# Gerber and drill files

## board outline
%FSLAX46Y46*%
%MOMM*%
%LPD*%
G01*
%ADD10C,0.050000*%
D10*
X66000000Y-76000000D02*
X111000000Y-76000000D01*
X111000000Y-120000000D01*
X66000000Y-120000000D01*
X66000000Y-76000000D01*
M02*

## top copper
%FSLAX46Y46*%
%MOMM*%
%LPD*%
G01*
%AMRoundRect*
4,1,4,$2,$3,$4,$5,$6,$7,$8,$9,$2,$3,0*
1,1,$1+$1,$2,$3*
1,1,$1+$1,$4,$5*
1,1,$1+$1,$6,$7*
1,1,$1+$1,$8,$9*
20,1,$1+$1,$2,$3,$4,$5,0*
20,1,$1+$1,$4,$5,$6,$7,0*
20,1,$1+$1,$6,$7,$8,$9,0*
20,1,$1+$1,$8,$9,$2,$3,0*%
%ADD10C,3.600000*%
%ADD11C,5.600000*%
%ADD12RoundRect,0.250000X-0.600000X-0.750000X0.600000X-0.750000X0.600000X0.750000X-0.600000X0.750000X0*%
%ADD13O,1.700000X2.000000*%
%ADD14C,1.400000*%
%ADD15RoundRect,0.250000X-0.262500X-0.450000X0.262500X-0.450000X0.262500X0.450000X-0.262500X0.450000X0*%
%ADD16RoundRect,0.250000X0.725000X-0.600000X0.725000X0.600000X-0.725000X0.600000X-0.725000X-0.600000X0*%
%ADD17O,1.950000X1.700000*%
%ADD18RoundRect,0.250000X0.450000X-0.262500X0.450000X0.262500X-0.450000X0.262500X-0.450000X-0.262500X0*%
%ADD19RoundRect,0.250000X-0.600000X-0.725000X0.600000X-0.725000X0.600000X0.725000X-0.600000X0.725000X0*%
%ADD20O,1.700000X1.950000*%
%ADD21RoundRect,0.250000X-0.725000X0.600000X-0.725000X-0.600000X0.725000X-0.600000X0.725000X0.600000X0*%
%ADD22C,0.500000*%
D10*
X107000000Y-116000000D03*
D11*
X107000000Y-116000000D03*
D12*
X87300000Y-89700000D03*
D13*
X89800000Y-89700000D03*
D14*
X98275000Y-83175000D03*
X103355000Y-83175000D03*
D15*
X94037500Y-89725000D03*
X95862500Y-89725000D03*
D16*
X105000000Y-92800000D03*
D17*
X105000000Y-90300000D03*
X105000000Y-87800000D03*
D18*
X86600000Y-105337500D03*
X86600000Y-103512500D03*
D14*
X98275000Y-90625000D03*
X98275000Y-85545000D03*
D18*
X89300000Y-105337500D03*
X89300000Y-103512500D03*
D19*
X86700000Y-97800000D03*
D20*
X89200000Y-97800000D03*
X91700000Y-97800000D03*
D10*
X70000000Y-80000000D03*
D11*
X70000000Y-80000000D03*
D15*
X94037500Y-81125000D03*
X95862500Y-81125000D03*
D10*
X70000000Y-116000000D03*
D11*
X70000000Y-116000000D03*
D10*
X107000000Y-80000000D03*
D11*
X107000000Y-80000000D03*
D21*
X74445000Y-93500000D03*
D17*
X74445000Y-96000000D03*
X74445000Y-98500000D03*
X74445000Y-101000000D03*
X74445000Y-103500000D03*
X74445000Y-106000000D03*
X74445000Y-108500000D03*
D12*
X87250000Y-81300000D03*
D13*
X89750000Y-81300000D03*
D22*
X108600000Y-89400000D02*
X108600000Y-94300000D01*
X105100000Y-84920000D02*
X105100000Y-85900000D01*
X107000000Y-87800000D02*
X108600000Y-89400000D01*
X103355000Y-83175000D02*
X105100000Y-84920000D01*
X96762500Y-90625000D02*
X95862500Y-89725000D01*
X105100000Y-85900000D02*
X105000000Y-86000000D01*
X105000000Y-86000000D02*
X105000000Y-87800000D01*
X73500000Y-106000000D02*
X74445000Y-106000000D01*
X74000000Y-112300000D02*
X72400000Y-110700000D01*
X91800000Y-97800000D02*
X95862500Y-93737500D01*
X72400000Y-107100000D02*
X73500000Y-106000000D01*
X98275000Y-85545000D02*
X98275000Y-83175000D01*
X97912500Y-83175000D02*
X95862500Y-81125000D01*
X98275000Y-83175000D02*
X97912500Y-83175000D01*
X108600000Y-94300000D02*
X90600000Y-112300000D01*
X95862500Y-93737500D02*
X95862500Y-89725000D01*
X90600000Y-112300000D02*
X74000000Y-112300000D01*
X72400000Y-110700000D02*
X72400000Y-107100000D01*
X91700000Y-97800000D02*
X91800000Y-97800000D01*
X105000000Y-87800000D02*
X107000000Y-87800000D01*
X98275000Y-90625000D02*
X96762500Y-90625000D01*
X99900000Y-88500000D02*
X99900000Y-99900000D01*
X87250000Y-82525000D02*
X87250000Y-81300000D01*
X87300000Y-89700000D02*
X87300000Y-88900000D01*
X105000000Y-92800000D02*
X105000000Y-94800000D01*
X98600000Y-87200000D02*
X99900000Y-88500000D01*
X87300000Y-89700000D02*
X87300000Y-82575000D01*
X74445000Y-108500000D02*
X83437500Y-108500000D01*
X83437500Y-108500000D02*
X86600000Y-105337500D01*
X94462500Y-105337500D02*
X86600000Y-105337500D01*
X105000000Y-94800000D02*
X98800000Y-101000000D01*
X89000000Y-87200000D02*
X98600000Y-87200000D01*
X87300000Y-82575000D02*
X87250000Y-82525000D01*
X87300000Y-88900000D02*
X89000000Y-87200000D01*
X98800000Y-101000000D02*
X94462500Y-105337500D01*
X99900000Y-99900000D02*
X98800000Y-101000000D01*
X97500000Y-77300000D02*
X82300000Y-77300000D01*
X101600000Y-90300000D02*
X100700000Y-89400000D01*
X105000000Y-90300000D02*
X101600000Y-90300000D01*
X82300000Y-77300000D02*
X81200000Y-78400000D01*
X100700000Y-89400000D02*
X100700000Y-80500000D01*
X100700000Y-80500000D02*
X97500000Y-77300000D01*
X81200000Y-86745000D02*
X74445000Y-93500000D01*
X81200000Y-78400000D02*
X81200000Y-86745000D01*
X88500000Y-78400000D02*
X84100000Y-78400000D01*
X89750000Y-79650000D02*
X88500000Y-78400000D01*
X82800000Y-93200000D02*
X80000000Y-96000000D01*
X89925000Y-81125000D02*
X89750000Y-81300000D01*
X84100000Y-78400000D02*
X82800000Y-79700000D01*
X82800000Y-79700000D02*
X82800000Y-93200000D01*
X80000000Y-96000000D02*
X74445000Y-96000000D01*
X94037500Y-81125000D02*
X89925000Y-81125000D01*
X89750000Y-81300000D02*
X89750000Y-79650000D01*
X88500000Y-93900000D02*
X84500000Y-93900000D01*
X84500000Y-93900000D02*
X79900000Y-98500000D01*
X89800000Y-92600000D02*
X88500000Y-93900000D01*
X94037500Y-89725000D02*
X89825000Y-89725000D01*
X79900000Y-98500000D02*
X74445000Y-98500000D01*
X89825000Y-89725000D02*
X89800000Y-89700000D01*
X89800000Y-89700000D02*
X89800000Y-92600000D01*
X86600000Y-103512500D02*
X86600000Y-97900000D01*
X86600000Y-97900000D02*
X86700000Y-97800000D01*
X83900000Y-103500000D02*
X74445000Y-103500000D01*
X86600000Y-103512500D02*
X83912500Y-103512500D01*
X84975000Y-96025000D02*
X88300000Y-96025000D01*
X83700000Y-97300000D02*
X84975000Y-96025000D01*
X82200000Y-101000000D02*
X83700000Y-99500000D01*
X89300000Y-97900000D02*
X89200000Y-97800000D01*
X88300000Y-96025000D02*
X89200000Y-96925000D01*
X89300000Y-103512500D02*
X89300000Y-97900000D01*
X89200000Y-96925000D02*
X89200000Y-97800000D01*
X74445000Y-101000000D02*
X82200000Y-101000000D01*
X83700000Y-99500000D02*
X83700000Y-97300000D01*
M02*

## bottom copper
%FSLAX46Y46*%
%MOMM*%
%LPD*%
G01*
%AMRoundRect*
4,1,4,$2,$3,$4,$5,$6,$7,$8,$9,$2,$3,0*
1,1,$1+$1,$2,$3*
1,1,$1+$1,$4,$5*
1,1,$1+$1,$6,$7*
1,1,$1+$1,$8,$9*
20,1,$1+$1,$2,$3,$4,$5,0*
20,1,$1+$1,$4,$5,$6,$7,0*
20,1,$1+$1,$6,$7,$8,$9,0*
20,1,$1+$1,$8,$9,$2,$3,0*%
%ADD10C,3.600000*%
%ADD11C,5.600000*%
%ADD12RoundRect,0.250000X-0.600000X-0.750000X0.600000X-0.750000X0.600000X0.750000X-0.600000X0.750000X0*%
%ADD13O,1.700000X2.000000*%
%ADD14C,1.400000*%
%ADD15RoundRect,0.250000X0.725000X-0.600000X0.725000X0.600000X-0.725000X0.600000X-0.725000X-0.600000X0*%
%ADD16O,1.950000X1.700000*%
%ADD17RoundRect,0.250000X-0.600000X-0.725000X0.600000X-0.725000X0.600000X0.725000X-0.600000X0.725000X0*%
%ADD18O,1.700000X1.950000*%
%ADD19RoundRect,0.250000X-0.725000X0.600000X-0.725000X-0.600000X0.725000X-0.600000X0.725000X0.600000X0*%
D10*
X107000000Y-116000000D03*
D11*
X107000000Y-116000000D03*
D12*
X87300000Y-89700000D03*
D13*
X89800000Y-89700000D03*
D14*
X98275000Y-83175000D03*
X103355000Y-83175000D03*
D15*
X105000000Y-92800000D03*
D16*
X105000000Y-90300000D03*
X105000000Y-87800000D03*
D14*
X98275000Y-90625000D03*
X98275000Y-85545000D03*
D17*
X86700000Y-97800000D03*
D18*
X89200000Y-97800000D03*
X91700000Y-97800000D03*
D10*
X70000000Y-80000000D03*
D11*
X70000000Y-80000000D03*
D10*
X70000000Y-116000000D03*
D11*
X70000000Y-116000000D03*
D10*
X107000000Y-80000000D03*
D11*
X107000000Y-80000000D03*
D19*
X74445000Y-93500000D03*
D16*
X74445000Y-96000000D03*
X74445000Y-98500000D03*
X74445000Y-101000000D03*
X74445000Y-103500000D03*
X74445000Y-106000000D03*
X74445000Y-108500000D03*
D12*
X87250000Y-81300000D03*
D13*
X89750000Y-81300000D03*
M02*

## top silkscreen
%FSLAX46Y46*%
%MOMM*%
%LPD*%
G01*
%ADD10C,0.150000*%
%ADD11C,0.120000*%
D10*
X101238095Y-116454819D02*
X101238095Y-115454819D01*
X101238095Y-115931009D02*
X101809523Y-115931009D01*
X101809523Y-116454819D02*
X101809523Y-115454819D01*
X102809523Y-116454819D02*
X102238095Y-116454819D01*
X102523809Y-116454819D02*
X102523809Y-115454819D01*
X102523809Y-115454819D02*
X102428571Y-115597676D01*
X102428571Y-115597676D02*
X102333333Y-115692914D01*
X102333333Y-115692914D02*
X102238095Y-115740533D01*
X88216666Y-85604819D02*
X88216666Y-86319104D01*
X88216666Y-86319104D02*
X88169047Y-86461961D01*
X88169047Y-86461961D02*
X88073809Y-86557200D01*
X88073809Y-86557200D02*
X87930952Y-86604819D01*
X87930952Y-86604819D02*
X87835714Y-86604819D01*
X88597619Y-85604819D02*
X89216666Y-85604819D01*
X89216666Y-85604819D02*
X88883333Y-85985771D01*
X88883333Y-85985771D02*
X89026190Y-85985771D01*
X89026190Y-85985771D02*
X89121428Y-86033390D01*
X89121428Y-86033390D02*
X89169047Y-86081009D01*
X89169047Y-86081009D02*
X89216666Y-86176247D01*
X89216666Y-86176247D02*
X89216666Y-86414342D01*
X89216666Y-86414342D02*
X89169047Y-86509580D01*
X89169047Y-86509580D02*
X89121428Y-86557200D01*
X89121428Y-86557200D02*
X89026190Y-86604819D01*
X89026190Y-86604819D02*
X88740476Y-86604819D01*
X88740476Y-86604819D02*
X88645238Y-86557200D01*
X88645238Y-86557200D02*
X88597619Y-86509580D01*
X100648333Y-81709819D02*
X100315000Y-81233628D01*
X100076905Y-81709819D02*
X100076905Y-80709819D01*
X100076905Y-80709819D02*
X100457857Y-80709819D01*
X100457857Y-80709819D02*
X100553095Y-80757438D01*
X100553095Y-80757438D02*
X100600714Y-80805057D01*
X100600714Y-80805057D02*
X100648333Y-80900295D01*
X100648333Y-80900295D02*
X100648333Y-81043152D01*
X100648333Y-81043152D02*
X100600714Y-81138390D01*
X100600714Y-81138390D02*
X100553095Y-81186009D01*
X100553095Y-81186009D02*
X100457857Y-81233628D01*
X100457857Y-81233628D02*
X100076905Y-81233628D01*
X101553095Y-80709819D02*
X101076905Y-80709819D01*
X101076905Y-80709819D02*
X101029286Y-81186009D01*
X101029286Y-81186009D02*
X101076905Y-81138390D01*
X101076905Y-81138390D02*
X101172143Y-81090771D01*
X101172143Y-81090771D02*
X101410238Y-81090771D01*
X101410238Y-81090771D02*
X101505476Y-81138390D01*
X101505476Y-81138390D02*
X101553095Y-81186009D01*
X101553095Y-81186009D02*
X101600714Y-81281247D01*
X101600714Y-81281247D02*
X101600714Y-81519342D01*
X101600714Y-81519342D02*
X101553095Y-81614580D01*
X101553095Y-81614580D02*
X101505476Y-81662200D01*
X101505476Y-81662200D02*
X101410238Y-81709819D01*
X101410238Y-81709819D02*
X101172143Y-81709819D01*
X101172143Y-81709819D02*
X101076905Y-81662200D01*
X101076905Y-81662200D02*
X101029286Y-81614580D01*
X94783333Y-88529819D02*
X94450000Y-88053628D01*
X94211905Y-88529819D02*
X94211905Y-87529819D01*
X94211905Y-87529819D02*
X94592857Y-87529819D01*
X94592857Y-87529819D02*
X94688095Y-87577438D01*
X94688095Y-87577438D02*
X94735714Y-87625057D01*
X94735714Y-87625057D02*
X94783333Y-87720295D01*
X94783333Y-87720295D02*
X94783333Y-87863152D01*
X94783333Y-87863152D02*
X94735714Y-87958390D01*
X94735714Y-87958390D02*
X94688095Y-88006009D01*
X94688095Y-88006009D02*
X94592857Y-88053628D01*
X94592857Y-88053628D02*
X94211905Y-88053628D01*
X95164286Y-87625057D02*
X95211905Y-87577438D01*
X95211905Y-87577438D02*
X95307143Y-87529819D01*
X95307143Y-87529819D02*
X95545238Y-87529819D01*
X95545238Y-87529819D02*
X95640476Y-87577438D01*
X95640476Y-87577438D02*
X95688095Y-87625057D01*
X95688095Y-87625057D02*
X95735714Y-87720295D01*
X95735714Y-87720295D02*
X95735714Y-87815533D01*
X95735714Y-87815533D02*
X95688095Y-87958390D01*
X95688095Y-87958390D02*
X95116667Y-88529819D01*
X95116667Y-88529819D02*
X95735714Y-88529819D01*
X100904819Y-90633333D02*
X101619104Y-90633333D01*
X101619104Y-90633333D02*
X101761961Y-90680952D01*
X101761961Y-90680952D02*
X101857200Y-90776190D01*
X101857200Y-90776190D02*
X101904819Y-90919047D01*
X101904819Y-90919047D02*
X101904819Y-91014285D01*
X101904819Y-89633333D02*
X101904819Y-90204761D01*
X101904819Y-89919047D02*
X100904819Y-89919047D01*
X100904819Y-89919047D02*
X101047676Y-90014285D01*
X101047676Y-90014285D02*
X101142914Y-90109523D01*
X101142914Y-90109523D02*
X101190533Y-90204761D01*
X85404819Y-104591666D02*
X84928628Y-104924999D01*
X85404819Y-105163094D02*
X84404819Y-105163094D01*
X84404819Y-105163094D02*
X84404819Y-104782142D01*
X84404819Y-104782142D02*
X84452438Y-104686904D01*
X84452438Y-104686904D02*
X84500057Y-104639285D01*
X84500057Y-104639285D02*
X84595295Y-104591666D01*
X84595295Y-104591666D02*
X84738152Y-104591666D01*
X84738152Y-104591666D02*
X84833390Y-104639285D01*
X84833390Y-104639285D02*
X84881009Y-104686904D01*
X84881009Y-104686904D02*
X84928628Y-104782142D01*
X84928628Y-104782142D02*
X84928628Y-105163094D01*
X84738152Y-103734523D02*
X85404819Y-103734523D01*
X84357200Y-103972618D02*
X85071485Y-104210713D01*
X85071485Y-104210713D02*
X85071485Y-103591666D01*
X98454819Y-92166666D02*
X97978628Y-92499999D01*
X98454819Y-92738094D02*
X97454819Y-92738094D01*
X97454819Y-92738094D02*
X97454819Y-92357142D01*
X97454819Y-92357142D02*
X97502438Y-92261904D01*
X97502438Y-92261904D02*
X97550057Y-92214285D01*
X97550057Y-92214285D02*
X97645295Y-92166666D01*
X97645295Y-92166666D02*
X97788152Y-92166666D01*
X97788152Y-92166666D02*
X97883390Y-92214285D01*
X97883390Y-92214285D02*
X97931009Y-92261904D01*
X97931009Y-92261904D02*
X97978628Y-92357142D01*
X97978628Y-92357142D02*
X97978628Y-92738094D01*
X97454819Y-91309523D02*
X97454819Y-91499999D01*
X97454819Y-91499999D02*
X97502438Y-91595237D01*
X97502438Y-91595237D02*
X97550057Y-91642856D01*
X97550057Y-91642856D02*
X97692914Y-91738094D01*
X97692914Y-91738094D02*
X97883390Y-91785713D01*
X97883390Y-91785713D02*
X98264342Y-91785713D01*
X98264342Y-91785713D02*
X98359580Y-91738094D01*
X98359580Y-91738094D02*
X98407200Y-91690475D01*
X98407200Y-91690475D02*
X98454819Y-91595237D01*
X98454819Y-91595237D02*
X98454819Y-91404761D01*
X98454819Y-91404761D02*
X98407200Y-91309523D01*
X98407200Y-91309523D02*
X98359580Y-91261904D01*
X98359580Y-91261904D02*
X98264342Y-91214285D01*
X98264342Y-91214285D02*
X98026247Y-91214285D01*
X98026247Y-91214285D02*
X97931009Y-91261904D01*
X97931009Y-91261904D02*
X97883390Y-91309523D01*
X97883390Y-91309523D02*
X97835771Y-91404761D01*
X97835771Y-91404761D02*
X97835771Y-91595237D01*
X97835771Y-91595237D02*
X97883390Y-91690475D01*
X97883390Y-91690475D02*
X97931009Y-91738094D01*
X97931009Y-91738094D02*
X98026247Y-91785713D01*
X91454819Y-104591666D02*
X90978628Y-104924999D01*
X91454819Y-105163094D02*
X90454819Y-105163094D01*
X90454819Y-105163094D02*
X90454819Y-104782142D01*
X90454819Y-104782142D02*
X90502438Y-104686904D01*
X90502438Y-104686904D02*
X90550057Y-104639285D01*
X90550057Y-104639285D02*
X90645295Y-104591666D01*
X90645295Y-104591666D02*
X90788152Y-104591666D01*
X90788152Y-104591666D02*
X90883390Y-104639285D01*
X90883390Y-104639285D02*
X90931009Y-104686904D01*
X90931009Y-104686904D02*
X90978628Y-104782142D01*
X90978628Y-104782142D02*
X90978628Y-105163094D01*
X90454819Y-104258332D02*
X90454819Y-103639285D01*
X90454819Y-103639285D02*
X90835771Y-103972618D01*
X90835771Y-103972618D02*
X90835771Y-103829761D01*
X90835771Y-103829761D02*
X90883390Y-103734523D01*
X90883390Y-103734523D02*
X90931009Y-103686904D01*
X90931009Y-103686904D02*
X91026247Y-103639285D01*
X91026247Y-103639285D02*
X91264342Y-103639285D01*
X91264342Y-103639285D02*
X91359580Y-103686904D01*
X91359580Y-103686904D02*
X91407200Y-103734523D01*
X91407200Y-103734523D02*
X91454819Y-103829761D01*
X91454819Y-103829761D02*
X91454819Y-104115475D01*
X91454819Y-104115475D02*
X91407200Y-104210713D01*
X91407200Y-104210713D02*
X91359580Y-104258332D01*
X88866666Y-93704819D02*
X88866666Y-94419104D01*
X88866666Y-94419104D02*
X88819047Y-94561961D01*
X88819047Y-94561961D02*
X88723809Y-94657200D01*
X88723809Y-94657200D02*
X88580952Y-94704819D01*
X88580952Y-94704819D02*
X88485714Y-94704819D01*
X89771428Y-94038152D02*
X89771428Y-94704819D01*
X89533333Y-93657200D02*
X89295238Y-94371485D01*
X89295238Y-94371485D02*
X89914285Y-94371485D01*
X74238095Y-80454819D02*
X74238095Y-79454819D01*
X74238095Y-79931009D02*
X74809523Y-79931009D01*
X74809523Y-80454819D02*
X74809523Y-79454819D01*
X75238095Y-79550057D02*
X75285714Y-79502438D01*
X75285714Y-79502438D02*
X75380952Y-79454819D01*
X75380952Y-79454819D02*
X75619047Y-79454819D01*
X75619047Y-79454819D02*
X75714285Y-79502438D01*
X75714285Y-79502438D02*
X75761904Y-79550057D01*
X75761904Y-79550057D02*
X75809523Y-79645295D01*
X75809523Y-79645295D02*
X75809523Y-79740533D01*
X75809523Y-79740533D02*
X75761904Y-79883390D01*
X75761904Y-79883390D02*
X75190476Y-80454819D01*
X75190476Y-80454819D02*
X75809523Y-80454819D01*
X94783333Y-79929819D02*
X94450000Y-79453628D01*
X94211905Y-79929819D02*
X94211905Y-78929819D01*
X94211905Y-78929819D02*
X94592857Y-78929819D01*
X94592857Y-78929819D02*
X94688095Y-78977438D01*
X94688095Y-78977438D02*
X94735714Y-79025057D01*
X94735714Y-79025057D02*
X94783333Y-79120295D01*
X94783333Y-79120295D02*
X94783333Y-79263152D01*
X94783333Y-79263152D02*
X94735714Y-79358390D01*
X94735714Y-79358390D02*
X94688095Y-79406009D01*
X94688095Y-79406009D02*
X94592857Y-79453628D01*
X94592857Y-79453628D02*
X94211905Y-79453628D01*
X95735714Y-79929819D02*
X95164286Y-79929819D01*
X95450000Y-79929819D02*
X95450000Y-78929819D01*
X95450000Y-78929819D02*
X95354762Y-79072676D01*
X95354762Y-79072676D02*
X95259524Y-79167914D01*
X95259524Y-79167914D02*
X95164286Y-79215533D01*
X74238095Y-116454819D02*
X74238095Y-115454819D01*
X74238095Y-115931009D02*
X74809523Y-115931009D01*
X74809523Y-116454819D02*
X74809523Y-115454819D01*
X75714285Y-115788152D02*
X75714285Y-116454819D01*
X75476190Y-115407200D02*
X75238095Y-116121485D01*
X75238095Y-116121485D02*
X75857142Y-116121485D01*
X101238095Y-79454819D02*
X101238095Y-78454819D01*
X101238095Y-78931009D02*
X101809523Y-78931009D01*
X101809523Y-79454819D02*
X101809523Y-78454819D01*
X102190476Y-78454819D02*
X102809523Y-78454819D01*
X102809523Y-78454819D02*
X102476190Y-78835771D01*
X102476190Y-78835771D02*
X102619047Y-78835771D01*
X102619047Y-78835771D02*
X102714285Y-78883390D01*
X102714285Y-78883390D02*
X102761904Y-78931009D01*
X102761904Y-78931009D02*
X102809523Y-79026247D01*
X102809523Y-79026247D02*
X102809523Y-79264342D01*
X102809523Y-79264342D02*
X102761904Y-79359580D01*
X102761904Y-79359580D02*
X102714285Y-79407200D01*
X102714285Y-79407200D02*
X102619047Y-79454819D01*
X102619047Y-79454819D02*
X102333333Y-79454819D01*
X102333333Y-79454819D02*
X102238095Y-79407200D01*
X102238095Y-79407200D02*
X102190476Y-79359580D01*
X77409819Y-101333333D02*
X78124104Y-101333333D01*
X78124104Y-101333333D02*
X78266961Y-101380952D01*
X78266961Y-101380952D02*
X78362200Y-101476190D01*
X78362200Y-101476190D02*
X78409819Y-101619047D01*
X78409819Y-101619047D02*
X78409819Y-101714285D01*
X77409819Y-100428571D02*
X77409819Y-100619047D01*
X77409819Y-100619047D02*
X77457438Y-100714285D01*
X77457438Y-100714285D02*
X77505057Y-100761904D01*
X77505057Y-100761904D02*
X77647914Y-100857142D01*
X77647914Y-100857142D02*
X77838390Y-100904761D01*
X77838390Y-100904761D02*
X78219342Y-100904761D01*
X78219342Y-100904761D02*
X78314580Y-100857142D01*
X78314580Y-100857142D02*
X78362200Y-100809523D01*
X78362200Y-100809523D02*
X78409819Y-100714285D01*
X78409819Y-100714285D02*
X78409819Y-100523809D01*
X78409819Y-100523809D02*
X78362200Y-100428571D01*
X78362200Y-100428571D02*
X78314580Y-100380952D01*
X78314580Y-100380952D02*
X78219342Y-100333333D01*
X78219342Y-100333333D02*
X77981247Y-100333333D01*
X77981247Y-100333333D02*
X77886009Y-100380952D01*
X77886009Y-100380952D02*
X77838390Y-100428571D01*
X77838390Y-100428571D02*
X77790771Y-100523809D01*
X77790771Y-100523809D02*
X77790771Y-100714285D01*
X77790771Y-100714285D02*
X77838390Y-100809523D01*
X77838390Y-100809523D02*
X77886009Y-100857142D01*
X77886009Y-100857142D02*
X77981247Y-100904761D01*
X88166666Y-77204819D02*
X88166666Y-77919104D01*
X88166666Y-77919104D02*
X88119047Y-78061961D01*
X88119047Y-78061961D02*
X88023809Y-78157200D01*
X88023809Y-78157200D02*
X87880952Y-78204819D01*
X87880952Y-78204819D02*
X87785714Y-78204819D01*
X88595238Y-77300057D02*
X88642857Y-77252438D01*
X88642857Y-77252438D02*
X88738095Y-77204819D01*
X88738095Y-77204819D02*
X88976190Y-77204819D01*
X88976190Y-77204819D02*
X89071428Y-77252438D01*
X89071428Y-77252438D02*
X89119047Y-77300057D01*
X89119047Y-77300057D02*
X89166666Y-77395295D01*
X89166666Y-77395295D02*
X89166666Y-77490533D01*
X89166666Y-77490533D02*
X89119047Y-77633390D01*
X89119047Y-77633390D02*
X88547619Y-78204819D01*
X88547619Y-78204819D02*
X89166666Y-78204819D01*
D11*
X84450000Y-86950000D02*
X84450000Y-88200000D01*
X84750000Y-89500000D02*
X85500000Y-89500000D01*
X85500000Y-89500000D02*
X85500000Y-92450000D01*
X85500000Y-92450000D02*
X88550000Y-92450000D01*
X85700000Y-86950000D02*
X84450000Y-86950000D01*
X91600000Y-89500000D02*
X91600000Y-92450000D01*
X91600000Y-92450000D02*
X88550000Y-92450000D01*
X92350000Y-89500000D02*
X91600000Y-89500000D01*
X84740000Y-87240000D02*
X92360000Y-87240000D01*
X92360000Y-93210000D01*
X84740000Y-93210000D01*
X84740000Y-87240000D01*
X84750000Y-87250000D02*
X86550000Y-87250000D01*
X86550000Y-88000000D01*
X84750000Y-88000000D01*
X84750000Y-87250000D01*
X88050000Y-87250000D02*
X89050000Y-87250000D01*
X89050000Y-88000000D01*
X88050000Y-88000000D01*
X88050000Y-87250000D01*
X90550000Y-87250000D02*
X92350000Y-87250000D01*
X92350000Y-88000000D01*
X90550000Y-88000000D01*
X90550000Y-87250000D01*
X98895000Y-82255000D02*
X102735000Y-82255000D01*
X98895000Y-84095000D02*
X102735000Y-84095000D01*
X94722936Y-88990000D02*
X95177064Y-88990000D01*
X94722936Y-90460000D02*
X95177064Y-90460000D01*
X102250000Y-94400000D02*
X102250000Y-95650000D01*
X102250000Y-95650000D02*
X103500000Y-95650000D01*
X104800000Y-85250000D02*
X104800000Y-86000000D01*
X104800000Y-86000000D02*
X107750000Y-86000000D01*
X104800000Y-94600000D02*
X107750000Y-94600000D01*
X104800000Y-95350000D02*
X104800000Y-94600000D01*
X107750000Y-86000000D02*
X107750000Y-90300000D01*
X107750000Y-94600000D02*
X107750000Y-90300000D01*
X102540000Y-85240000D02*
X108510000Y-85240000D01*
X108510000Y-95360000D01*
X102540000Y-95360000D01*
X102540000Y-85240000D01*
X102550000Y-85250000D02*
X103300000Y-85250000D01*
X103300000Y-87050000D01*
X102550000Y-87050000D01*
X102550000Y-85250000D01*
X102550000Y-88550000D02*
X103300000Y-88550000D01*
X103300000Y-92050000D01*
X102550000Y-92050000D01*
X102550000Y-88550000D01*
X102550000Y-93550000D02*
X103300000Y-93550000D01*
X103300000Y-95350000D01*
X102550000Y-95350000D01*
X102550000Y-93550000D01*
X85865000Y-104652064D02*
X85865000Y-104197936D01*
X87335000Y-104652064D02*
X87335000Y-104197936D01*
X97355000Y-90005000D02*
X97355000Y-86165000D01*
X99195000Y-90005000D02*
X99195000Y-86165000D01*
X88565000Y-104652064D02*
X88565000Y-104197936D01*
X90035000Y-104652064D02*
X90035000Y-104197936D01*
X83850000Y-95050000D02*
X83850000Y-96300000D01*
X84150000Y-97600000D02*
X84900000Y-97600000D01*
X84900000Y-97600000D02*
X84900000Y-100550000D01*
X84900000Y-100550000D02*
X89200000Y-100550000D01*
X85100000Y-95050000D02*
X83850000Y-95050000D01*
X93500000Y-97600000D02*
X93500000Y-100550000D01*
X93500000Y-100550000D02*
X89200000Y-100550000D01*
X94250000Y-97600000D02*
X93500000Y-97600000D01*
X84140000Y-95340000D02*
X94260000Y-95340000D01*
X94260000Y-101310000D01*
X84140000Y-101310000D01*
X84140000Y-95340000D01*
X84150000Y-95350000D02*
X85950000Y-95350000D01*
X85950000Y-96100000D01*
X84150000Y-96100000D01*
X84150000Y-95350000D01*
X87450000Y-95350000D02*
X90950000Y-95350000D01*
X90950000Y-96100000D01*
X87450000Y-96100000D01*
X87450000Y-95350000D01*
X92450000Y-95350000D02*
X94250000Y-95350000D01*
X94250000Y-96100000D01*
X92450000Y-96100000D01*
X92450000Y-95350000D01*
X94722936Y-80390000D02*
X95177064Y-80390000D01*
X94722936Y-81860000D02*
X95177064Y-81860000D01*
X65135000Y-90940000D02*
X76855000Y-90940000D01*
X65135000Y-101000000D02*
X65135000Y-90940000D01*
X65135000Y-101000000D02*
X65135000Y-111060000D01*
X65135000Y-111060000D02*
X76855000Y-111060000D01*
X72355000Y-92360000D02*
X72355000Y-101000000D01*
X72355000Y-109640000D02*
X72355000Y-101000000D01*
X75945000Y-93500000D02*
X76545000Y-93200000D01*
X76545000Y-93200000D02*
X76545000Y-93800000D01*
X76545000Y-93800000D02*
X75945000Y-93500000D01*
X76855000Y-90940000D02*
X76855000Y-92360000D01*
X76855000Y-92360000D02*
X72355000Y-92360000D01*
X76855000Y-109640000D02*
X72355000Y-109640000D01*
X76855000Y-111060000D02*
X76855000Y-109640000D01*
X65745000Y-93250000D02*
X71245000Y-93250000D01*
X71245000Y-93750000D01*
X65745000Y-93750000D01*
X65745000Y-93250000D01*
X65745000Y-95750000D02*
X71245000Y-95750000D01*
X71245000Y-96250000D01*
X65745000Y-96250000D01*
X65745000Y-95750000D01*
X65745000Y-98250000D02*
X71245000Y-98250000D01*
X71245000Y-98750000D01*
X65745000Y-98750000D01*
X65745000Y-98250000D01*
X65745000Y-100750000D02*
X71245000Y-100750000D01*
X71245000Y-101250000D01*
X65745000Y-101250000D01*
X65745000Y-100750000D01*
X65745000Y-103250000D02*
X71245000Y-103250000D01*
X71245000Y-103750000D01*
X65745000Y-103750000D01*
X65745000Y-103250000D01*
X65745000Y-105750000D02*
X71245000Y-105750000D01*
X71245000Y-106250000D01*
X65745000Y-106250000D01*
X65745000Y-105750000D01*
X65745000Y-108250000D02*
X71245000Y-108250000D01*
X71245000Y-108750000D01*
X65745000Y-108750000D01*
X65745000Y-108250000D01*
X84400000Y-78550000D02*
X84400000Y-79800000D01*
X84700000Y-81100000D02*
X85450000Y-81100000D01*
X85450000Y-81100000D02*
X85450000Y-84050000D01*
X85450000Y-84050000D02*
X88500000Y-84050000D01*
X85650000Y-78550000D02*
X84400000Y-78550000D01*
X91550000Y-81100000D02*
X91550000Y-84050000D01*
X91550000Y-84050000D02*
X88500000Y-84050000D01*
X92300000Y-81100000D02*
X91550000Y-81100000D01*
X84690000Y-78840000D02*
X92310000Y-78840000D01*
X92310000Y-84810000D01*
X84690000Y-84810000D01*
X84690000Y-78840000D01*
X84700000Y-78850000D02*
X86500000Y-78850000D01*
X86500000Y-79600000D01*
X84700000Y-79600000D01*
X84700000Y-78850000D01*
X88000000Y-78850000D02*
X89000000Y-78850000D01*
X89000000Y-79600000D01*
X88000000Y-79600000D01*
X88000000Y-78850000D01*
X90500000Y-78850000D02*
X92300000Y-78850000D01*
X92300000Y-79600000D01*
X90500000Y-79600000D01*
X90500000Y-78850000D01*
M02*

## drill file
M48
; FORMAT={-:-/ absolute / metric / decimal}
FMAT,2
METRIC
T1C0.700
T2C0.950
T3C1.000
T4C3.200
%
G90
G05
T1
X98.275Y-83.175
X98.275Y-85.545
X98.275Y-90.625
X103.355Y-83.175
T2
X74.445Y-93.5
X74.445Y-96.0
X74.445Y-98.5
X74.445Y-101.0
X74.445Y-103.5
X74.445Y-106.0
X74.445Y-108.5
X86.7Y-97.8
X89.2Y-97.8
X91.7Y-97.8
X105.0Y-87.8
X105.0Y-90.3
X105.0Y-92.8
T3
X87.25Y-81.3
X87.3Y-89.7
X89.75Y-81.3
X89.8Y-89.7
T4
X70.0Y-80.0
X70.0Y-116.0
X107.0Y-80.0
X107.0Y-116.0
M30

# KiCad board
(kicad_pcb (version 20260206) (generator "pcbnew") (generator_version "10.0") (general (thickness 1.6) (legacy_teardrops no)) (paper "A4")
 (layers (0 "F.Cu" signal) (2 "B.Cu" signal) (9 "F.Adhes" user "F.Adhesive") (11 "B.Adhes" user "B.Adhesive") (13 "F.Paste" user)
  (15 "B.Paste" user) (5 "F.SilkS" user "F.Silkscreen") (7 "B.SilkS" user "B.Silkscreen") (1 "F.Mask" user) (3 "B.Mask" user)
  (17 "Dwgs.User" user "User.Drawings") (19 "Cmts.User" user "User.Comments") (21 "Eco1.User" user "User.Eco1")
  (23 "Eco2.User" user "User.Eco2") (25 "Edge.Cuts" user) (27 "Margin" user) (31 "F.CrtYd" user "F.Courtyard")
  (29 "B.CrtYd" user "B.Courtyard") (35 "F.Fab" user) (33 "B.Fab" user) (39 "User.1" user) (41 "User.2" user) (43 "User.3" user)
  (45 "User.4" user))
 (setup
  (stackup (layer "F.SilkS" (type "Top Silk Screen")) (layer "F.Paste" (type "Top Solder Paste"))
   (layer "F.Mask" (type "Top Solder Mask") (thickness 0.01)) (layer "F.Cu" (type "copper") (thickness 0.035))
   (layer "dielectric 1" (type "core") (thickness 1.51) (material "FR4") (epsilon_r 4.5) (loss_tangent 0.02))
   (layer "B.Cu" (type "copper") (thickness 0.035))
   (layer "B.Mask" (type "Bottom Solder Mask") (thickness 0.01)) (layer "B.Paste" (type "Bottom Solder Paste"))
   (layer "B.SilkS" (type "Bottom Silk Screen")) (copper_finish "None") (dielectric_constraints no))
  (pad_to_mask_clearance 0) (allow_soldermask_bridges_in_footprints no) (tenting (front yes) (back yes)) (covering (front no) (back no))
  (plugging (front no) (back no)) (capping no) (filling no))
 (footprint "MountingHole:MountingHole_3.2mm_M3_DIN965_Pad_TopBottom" (layer "F.Cu") (at 107 116)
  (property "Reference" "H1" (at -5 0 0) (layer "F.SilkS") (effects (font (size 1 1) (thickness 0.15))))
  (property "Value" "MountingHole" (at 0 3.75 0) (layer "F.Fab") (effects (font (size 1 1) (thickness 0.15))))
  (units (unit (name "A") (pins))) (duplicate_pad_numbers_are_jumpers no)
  (pad "1" thru_hole circle (at 0 0) (size 3.6 3.6) (drill 3.2) (layers "*.Cu" "*.Mask") (remove_unused_layers no) (zone_connect 2))
  (pad "1" connect circle (at 0 0) (size 5.6 5.6) (layers "F.Cu" "F.Mask") (zone_connect 2))
  (pad "1" connect circle (at 0 0) (size 5.6 5.6) (layers "B.Cu" "B.Mask") (zone_connect 2)))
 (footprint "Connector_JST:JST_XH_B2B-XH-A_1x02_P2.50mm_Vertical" (layer "F.Cu") (at 87.3 89.7)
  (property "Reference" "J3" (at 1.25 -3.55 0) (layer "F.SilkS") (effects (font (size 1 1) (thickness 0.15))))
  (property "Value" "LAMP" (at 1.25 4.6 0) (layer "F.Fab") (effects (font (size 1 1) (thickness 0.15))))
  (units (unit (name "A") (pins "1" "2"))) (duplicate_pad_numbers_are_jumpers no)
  (fp_line (start -2.85 -2.75) (end -2.85 -1.5) (stroke (width 0.12) (type solid)) (layer "F.SilkS"))
  (fp_line (start -2.55 -0.2) (end -1.8 -0.2) (stroke (width 0.12) (type solid)) (layer "F.SilkS"))
  (fp_line (start -1.8 -0.2) (end -1.8 2.75) (stroke (width 0.12) (type solid)) (layer "F.SilkS"))
  (fp_line (start -1.8 2.75) (end 1.25 2.75) (stroke (width 0.12) (type solid)) (layer "F.SilkS"))
  (fp_line (start -1.6 -2.75) (end -2.85 -2.75) (stroke (width 0.12) (type solid)) (layer "F.SilkS"))
  (fp_line (start 4.3 -0.2) (end 4.3 2.75) (stroke (width 0.12) (type solid)) (layer "F.SilkS"))
  (fp_line (start 4.3 2.75) (end 1.25 2.75) (stroke (width 0.12) (type solid)) (layer "F.SilkS"))
  (fp_line (start 5.05 -0.2) (end 4.3 -0.2) (stroke (width 0.12) (type solid)) (layer "F.SilkS"))
  (fp_rect (start -2.56 -2.46) (end 5.06 3.51) (stroke (width 0.12) (type solid)) (fill no) (layer "F.SilkS"))
  (fp_rect (start -2.55 -2.45) (end -0.75 -1.7) (stroke (width 0.12) (type solid)) (fill no) (layer "F.SilkS"))
  (fp_rect (start 0.75 -2.45) (end 1.75 -1.7) (stroke (width 0.12) (type solid)) (fill no) (layer "F.SilkS"))
  (fp_rect (start 3.25 -2.45) (end 5.05 -1.7) (stroke (width 0.12) (type solid)) (fill no) (layer "F.SilkS"))
  (pad "1" thru_hole roundrect (at 0 0) (size 1.7 2) (drill 1) (layers "*.Cu" "*.Mask") (remove_unused_layers no)
   (roundrect_rratio 0.147059) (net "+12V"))
  (pad "2" thru_hole oval (at 2.5 0) (size 1.7 2) (drill 1) (layers "*.Cu" "*.Mask") (remove_unused_layers no) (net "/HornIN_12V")))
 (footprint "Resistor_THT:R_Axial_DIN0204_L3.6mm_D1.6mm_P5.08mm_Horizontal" (layer "F.Cu") (at 98.275 83.175)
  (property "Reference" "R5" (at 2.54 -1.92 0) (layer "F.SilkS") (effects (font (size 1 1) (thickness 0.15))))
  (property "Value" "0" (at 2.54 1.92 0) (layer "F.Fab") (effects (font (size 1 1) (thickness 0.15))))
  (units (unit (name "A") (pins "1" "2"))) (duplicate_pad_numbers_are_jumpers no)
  (fp_line (start 0.62 -0.92) (end 4.46 -0.92) (stroke (width 0.12) (type solid)) (layer "F.SilkS"))
  (fp_line (start 0.62 0.92) (end 4.46 0.92) (stroke (width 0.12) (type solid)) (layer "F.SilkS"))
  (pad "1" thru_hole circle (at 0 0) (size 1.4 1.4) (drill 0.7) (layers "*.Cu" "*.Mask") (remove_unused_layers no) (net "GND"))
  (pad "2" thru_hole circle (at 5.08 0) (size 1.4 1.4) (drill 0.7) (layers "*.Cu" "*.Mask") (remove_unused_layers no) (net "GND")))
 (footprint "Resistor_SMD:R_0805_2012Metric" (layer "F.Cu") (at 94.95 89.725)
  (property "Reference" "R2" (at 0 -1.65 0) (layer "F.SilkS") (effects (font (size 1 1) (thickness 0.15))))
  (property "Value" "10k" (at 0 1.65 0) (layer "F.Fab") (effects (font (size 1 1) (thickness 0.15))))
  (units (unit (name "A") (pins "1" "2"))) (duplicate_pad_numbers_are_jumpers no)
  (fp_line (start -0.227064 -0.735) (end 0.227064 -0.735) (stroke (width 0.12) (type solid)) (layer "F.SilkS"))
  (fp_line (start -0.227064 0.735) (end 0.227064 0.735) (stroke (width 0.12) (type solid)) (layer "F.SilkS"))
  (pad "1" smd roundrect (at -0.9125 0) (size 1.025 1.4) (layers "F.Cu" "F.Mask" "F.Paste") (roundrect_rratio 0.243902) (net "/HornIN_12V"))
  (pad "2" smd roundrect (at 0.9125 0) (size 1.025 1.4) (layers "F.Cu" "F.Mask" "F.Paste") (roundrect_rratio 0.243902) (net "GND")))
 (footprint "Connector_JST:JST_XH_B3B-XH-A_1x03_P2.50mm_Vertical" (layer "F.Cu") (at 105 92.8 90)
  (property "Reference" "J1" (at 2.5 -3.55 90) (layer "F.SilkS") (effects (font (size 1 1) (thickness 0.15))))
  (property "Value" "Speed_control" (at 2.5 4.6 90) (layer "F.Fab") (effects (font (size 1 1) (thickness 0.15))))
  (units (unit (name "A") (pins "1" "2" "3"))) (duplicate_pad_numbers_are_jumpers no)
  (fp_line (start -1.6 -2.75) (end -2.85 -2.75) (stroke (width 0.12) (type solid)) (layer "F.SilkS"))
  (fp_line (start -2.85 -2.75) (end -2.85 -1.5) (stroke (width 0.12) (type solid)) (layer "F.SilkS"))
  (fp_line (start 7.55 -0.2) (end 6.8 -0.2) (stroke (width 0.12) (type solid)) (layer "F.SilkS"))
  (fp_line (start 6.8 -0.2) (end 6.8 2.75) (stroke (width 0.12) (type solid)) (layer "F.SilkS"))
  (fp_line (start -1.8 -0.2) (end -1.8 2.75) (stroke (width 0.12) (type solid)) (layer "F.SilkS"))
  (fp_line (start -2.55 -0.2) (end -1.8 -0.2) (stroke (width 0.12) (type solid)) (layer "F.SilkS"))
  (fp_line (start 6.8 2.75) (end 2.5 2.75) (stroke (width 0.12) (type solid)) (layer "F.SilkS"))
  (fp_line (start -1.8 2.75) (end 2.5 2.75) (stroke (width 0.12) (type solid)) (layer "F.SilkS"))
  (fp_rect (start -2.56 -2.46) (end 7.56 3.51) (stroke (width 0.12) (type solid)) (fill no) (layer "F.SilkS"))
  (fp_rect (start 5.75 -2.45) (end 7.55 -1.7) (stroke (width 0.12) (type solid)) (fill no) (layer "F.SilkS"))
  (fp_rect (start 0.75 -2.45) (end 4.25 -1.7) (stroke (width 0.12) (type solid)) (fill no) (layer "F.SilkS"))
  (fp_rect (start -2.55 -2.45) (end -0.75 -1.7) (stroke (width 0.12) (type solid)) (fill no) (layer "F.SilkS"))
  (pad "1" thru_hole roundrect (at 0 0 90) (size 1.7 1.95) (drill 0.95) (layers "*.Cu" "*.Mask") (remove_unused_layers no)
   (roundrect_rratio 0.147059) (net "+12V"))
  (pad "2" thru_hole oval (at 2.5 0 90) (size 1.7 1.95) (drill 0.95) (layers "*.Cu" "*.Mask") (remove_unused_layers no)
   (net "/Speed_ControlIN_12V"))
  (pad "3" thru_hole oval (at 5 0 90) (size 1.7 1.95) (drill 0.95) (layers "*.Cu" "*.Mask") (remove_unused_layers no) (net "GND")))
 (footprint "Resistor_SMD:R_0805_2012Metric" (layer "F.Cu") (at 86.6 104.425 90)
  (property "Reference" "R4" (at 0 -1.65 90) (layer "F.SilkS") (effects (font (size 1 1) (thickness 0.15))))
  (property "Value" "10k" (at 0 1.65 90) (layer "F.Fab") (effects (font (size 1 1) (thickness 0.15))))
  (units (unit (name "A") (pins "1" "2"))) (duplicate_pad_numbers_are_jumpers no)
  (fp_line (start -0.227064 -0.735) (end 0.227064 -0.735) (stroke (width 0.12) (type solid)) (layer "F.SilkS"))
  (fp_line (start -0.227064 0.735) (end 0.227064 0.735) (stroke (width 0.12) (type solid)) (layer "F.SilkS"))
  (pad "1" smd roundrect (at -0.9125 0 90) (size 1.025 1.4) (layers "F.Cu" "F.Mask" "F.Paste") (roundrect_rratio 0.243902) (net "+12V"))
  (pad "2" smd roundrect (at 0.9125 0 90) (size 1.025 1.4) (layers "F.Cu" "F.Mask" "F.Paste") (roundrect_rratio 0.243902)
   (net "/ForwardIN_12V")))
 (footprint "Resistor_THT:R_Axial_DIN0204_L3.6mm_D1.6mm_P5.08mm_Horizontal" (layer "F.Cu") (at 98.275 90.625 90)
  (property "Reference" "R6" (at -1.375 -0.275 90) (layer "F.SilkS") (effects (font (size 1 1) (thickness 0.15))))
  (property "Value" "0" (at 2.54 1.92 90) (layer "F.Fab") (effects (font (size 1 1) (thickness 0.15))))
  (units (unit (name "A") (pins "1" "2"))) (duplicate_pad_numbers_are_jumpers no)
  (fp_line (start 0.62 -0.92) (end 4.46 -0.92) (stroke (width 0.12) (type solid)) (layer "F.SilkS"))
  (fp_line (start 0.62 0.92) (end 4.46 0.92) (stroke (width 0.12) (type solid)) (layer "F.SilkS"))
  (pad "1" thru_hole circle (at 0 0 90) (size 1.4 1.4) (drill 0.7) (layers "*.Cu" "*.Mask") (remove_unused_layers no) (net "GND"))
  (pad "2" thru_hole circle (at 5.08 0 90) (size 1.4 1.4) (drill 0.7) (layers "*.Cu" "*.Mask") (remove_unused_layers no) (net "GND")))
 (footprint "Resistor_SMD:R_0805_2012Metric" (layer "F.Cu") (at 89.3 104.425 90)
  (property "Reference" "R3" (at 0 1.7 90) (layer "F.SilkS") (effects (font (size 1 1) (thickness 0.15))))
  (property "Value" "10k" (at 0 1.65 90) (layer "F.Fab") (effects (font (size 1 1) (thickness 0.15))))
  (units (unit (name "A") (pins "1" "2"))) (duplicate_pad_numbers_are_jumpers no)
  (fp_line (start -0.227064 -0.735) (end 0.227064 -0.735) (stroke (width 0.12) (type solid)) (layer "F.SilkS"))
  (fp_line (start -0.227064 0.735) (end 0.227064 0.735) (stroke (width 0.12) (type solid)) (layer "F.SilkS"))
  (pad "1" smd roundrect (at -0.9125 0 90) (size 1.025 1.4) (layers "F.Cu" "F.Mask" "F.Paste") (roundrect_rratio 0.243902) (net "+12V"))
  (pad "2" smd roundrect (at 0.9125 0 90) (size 1.025 1.4) (layers "F.Cu" "F.Mask" "F.Paste") (roundrect_rratio 0.243902)
   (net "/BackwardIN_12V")))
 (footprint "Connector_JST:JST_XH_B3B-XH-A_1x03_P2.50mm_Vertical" (layer "F.Cu") (at 86.7 97.8)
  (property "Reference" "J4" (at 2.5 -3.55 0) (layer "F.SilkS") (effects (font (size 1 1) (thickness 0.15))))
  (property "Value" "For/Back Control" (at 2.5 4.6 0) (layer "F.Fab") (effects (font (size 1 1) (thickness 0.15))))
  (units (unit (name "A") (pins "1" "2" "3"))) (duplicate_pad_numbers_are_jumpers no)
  (fp_line (start -2.85 -2.75) (end -2.85 -1.5) (stroke (width 0.12) (type solid)) (layer "F.SilkS"))
  (fp_line (start -2.55 -0.2) (end -1.8 -0.2) (stroke (width 0.12) (type solid)) (layer "F.SilkS"))
  (fp_line (start -1.8 -0.2) (end -1.8 2.75) (stroke (width 0.12) (type solid)) (layer "F.SilkS"))
  (fp_line (start -1.8 2.75) (end 2.5 2.75) (stroke (width 0.12) (type solid)) (layer "F.SilkS"))
  (fp_line (start -1.6 -2.75) (end -2.85 -2.75) (stroke (width 0.12) (type solid)) (layer "F.SilkS"))
  (fp_line (start 6.8 -0.2) (end 6.8 2.75) (stroke (width 0.12) (type solid)) (layer "F.SilkS"))
  (fp_line (start 6.8 2.75) (end 2.5 2.75) (stroke (width 0.12) (type solid)) (layer "F.SilkS"))
  (fp_line (start 7.55 -0.2) (end 6.8 -0.2) (stroke (width 0.12) (type solid)) (layer "F.SilkS"))
  (fp_rect (start -2.56 -2.46) (end 7.56 3.51) (stroke (width 0.12) (type solid)) (fill no) (layer "F.SilkS"))
  (fp_rect (start -2.55 -2.45) (end -0.75 -1.7) (stroke (width 0.12) (type solid)) (fill no) (layer "F.SilkS"))
  (fp_rect (start 0.75 -2.45) (end 4.25 -1.7) (stroke (width 0.12) (type solid)) (fill no) (layer "F.SilkS"))
  (fp_rect (start 5.75 -2.45) (end 7.55 -1.7) (stroke (width 0.12) (type solid)) (fill no) (layer "F.SilkS"))
  (pad "1" thru_hole roundrect (at 0 0) (size 1.7 1.95) (drill 0.95) (layers "*.Cu" "*.Mask") (remove_unused_layers no)
   (roundrect_rratio 0.147059) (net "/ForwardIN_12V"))
  (pad "2" thru_hole oval (at 2.5 0) (size 1.7 1.95) (drill 0.95) (layers "*.Cu" "*.Mask") (remove_unused_layers no) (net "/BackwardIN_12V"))
  (pad "3" thru_hole oval (at 5 0) (size 1.7 1.95) (drill 0.95) (layers "*.Cu" "*.Mask") (remove_unused_layers no) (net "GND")))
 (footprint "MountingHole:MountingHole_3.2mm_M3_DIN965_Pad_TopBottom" (layer "F.Cu") (at 70 80)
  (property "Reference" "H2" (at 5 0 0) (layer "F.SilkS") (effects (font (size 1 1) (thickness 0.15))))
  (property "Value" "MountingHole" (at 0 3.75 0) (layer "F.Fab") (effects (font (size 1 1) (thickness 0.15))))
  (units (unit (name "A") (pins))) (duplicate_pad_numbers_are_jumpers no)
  (pad "1" thru_hole circle (at 0 0) (size 3.6 3.6) (drill 3.2) (layers "*.Cu" "*.Mask") (remove_unused_layers no) (zone_connect 2))
  (pad "1" connect circle (at 0 0) (size 5.6 5.6) (layers "F.Cu" "F.Mask") (zone_connect 2))
  (pad "1" connect circle (at 0 0) (size 5.6 5.6) (layers "B.Cu" "B.Mask") (zone_connect 2)))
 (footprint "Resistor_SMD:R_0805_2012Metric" (layer "F.Cu") (at 94.95 81.125)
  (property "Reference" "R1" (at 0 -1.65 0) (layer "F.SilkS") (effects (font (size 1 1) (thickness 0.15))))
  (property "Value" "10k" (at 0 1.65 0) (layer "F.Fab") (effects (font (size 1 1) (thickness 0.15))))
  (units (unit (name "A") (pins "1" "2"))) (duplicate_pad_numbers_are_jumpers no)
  (fp_line (start -0.227064 -0.735) (end 0.227064 -0.735) (stroke (width 0.12) (type solid)) (layer "F.SilkS"))
  (fp_line (start -0.227064 0.735) (end 0.227064 0.735) (stroke (width 0.12) (type solid)) (layer "F.SilkS"))
  (pad "1" smd roundrect (at -0.9125 0) (size 1.025 1.4) (layers "F.Cu" "F.Mask" "F.Paste") (roundrect_rratio 0.243902) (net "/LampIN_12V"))
  (pad "2" smd roundrect (at 0.9125 0) (size 1.025 1.4) (layers "F.Cu" "F.Mask" "F.Paste") (roundrect_rratio 0.243902) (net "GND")))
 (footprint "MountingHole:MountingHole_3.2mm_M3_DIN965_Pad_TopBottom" (layer "F.Cu") (at 70 116)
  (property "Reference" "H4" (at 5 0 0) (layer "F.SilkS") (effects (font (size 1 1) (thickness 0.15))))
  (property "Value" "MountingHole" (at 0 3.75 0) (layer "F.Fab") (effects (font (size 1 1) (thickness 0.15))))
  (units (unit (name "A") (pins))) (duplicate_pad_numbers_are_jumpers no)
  (pad "1" thru_hole circle (at 0 0) (size 3.6 3.6) (drill 3.2) (layers "*.Cu" "*.Mask") (remove_unused_layers no) (zone_connect 2))
  (pad "1" connect circle (at 0 0) (size 5.6 5.6) (layers "F.Cu" "F.Mask") (zone_connect 2))
  (pad "1" connect circle (at 0 0) (size 5.6 5.6) (layers "B.Cu" "B.Mask") (zone_connect 2)))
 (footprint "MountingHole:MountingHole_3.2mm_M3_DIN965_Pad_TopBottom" (layer "F.Cu") (at 107 80)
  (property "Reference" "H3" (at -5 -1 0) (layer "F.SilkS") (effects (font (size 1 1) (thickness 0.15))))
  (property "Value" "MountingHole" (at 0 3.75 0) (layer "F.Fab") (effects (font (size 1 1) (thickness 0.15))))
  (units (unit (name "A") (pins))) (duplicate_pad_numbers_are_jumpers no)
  (pad "1" thru_hole circle (at 0 0) (size 3.6 3.6) (drill 3.2) (layers "*.Cu" "*.Mask") (remove_unused_layers no) (zone_connect 2))
  (pad "1" connect circle (at 0 0) (size 5.6 5.6) (layers "F.Cu" "F.Mask") (zone_connect 2))
  (pad "1" connect circle (at 0 0) (size 5.6 5.6) (layers "B.Cu" "B.Mask") (zone_connect 2)))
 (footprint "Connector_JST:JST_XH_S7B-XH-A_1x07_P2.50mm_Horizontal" (layer "F.Cu") (at 74.445 93.5 -90)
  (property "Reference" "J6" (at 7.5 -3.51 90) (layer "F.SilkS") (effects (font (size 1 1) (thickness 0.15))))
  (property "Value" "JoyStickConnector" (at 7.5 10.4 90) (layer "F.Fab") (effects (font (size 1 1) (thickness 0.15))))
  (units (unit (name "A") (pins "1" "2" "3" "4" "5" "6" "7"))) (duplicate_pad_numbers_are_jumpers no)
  (fp_line (start -2.56 9.31) (end -2.56 -2.41) (stroke (width 0.12) (type solid)) (layer "F.SilkS"))
  (fp_line (start 7.5 9.31) (end -2.56 9.31) (stroke (width 0.12) (type solid)) (layer "F.SilkS"))
  (fp_line (start 7.5 9.31) (end 17.56 9.31) (stroke (width 0.12) (type solid)) (layer "F.SilkS"))
  (fp_line (start 17.56 9.31) (end 17.56 -2.41) (stroke (width 0.12) (type solid)) (layer "F.SilkS"))
  (fp_line (start -1.14 2.09) (end 7.5 2.09) (stroke (width 0.12) (type solid)) (layer "F.SilkS"))
  (fp_line (start 16.14 2.09) (end 7.5 2.09) (stroke (width 0.12) (type solid)) (layer "F.SilkS"))
  (fp_line (start 0 -1.5) (end -0.3 -2.1) (stroke (width 0.12) (type solid)) (layer "F.SilkS"))
  (fp_line (start -0.3 -2.1) (end 0.3 -2.1) (stroke (width 0.12) (type solid)) (layer "F.SilkS"))
  (fp_line (start 0.3 -2.1) (end 0 -1.5) (stroke (width 0.12) (type solid)) (layer "F.SilkS"))
  (fp_line (start -2.56 -2.41) (end -1.14 -2.41) (stroke (width 0.12) (type solid)) (layer "F.SilkS"))
  (fp_line (start -1.14 -2.41) (end -1.14 2.09) (stroke (width 0.12) (type solid)) (layer "F.SilkS"))
  (fp_line (start 16.14 -2.41) (end 16.14 2.09) (stroke (width 0.12) (type solid)) (layer "F.SilkS"))
  (fp_line (start 17.56 -2.41) (end 16.14 -2.41) (stroke (width 0.12) (type solid)) (layer "F.SilkS"))
  (fp_rect (start -0.25 3.2) (end 0.25 8.7) (stroke (width 0.12) (type solid)) (fill no) (layer "F.SilkS"))
  (fp_rect (start 2.25 3.2) (end 2.75 8.7) (stroke (width 0.12) (type solid)) (fill no) (layer "F.SilkS"))
  (fp_rect (start 4.75 3.2) (end 5.25 8.7) (stroke (width 0.12) (type solid)) (fill no) (layer "F.SilkS"))
  (fp_rect (start 7.25 3.2) (end 7.75 8.7) (stroke (width 0.12) (type solid)) (fill no) (layer "F.SilkS"))
  (fp_rect (start 9.75 3.2) (end 10.25 8.7) (stroke (width 0.12) (type solid)) (fill no) (layer "F.SilkS"))
  (fp_rect (start 12.25 3.2) (end 12.75 8.7) (stroke (width 0.12) (type solid)) (fill no) (layer "F.SilkS"))
  (fp_rect (start 14.75 3.2) (end 15.25 8.7) (stroke (width 0.12) (type solid)) (fill no) (layer "F.SilkS"))
  (pad "1" thru_hole roundrect (at 0 0 270) (size 1.7 1.95) (drill 0.95) (layers "*.Cu" "*.Mask") (remove_unused_layers no)
   (roundrect_rratio 0.147059) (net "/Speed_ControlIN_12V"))
  (pad "2" thru_hole oval (at 2.5 0 270) (size 1.7 1.95) (drill 0.95) (layers "*.Cu" "*.Mask") (remove_unused_layers no) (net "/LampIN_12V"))
  (pad "3" thru_hole oval (at 5 0 270) (size 1.7 1.95) (drill 0.95) (layers "*.Cu" "*.Mask") (remove_unused_layers no) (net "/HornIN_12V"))
  (pad "4" thru_hole oval (at 7.5 0 270) (size 1.7 1.95) (drill 0.95) (layers "*.Cu" "*.Mask") (remove_unused_layers no)
   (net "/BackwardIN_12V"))
  (pad "5" thru_hole oval (at 10 0 270) (size 1.7 1.95) (drill 0.95) (layers "*.Cu" "*.Mask") (remove_unused_layers no)
   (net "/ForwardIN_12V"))
  (pad "6" thru_hole oval (at 12.5 0 270) (size 1.7 1.95) (drill 0.95) (layers "*.Cu" "*.Mask") (remove_unused_layers no) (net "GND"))
  (pad "7" thru_hole oval (at 15 0 270) (size 1.7 1.95) (drill 0.95) (layers "*.Cu" "*.Mask") (remove_unused_layers no) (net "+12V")))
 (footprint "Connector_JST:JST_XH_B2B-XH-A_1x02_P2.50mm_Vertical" (layer "F.Cu") (at 87.25 81.3)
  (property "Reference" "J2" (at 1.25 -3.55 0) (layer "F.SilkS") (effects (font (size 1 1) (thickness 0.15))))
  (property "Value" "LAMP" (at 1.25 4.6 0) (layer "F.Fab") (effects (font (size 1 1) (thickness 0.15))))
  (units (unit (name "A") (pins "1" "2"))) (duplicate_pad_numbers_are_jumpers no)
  (fp_line (start -2.85 -2.75) (end -2.85 -1.5) (stroke (width 0.12) (type solid)) (layer "F.SilkS"))
  (fp_line (start -2.55 -0.2) (end -1.8 -0.2) (stroke (width 0.12) (type solid)) (layer "F.SilkS"))
  (fp_line (start -1.8 -0.2) (end -1.8 2.75) (stroke (width 0.12) (type solid)) (layer "F.SilkS"))
  (fp_line (start -1.8 2.75) (end 1.25 2.75) (stroke (width 0.12) (type solid)) (layer "F.SilkS"))
  (fp_line (start -1.6 -2.75) (end -2.85 -2.75) (stroke (width 0.12) (type solid)) (layer "F.SilkS"))
  (fp_line (start 4.3 -0.2) (end 4.3 2.75) (stroke (width 0.12) (type solid)) (layer "F.SilkS"))
  (fp_line (start 4.3 2.75) (end 1.25 2.75) (stroke (width 0.12) (type solid)) (layer "F.SilkS"))
  (fp_line (start 5.05 -0.2) (end 4.3 -0.2) (stroke (width 0.12) (type solid)) (layer "F.SilkS"))
  (fp_rect (start -2.56 -2.46) (end 5.06 3.51) (stroke (width 0.12) (type solid)) (fill no) (layer "F.SilkS"))
  (fp_rect (start -2.55 -2.45) (end -0.75 -1.7) (stroke (width 0.12) (type solid)) (fill no) (layer "F.SilkS"))
  (fp_rect (start 0.75 -2.45) (end 1.75 -1.7) (stroke (width 0.12) (type solid)) (fill no) (layer "F.SilkS"))
  (fp_rect (start 3.25 -2.45) (end 5.05 -1.7) (stroke (width 0.12) (type solid)) (fill no) (layer "F.SilkS"))
  (pad "1" thru_hole roundrect (at 0 0) (size 1.7 2) (drill 1) (layers "*.Cu" "*.Mask") (remove_unused_layers no)
   (roundrect_rratio 0.147059) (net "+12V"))
  (pad "2" thru_hole oval (at 2.5 0) (size 1.7 2) (drill 1) (layers "*.Cu" "*.Mask") (remove_unused_layers no) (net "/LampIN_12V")))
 (gr_rect (start 66 76) (end 111 120) (stroke (width 0.05) (type default)) (fill no) (layer "Edge.Cuts"))
 (segment (start 108.6 89.4) (end 108.6 94.3) (width 0.5) (layer "F.Cu") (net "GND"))
 (segment (start 105.1 84.92) (end 105.1 85.9) (width 0.5) (layer "F.Cu") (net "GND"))
 (segment (start 107 87.8) (end 108.6 89.4) (width 0.5) (layer "F.Cu") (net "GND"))
 (segment (start 103.355 83.175) (end 105.1 84.92) (width 0.5) (layer "F.Cu") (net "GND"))
 (segment (start 96.7625 90.625) (end 95.8625 89.725) (width 0.5) (layer "F.Cu") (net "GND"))
 (segment (start 105.1 85.9) (end 105 86) (width 0.5) (layer "F.Cu") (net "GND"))
 (segment (start 105 86) (end 105 87.8) (width 0.5) (layer "F.Cu") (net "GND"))
 (segment (start 73.5 106) (end 74.445 106) (width 0.5) (layer "F.Cu") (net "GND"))
 (segment (start 74 112.3) (end 72.4 110.7) (width 0.5) (layer "F.Cu") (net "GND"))
 (segment (start 91.8 97.8) (end 95.8625 93.7375) (width 0.5) (layer "F.Cu") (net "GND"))
 (segment (start 72.4 107.1) (end 73.5 106) (width 0.5) (layer "F.Cu") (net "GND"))
 (segment (start 98.275 85.545) (end 98.275 83.175) (width 0.5) (layer "F.Cu") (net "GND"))
 (segment (start 97.9125 83.175) (end 95.8625 81.125) (width 0.5) (layer "F.Cu") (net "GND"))
 (segment (start 98.275 83.175) (end 97.9125 83.175) (width 0.5) (layer "F.Cu") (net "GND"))
 (segment (start 108.6 94.3) (end 90.6 112.3) (width 0.5) (layer "F.Cu") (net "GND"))
 (segment (start 95.8625 93.7375) (end 95.8625 89.725) (width 0.5) (layer "F.Cu") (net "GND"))
 (segment (start 90.6 112.3) (end 74 112.3) (width 0.5) (layer "F.Cu") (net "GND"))
 (segment (start 72.4 110.7) (end 72.4 107.1) (width 0.5) (layer "F.Cu") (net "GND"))
 (segment (start 91.7 97.8) (end 91.8 97.8) (width 0.5) (layer "F.Cu") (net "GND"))
 (segment (start 105 87.8) (end 107 87.8) (width 0.5) (layer "F.Cu") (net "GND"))
 (segment (start 98.275 90.625) (end 96.7625 90.625) (width 0.5) (layer "F.Cu") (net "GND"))
 (segment (start 99.9 88.5) (end 99.9 99.9) (width 0.5) (layer "F.Cu") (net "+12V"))
 (segment (start 87.25 82.525) (end 87.25 81.3) (width 0.5) (layer "F.Cu") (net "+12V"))
 (segment (start 87.3 89.7) (end 87.3 88.9) (width 0.5) (layer "F.Cu") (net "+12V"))
 (segment (start 105 92.8) (end 105 94.8) (width 0.5) (layer "F.Cu") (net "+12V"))
 (segment (start 98.6 87.2) (end 99.9 88.5) (width 0.5) (layer "F.Cu") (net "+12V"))
 (segment (start 87.3 89.7) (end 87.3 82.575) (width 0.5) (layer "F.Cu") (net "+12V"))
 (segment (start 74.445 108.5) (end 83.4375 108.5) (width 0.5) (layer "F.Cu") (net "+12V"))
 (segment (start 83.4375 108.5) (end 86.6 105.3375) (width 0.5) (layer "F.Cu") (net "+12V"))
 (segment (start 94.4625 105.3375) (end 86.6 105.3375) (width 0.5) (layer "F.Cu") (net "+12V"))
 (segment (start 105 94.8) (end 98.8 101) (width 0.5) (layer "F.Cu") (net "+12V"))
 (segment (start 89 87.2) (end 98.6 87.2) (width 0.5) (layer "F.Cu") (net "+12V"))
 (segment (start 87.3 82.575) (end 87.25 82.525) (width 0.5) (layer "F.Cu") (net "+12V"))
 (segment (start 87.3 88.9) (end 89 87.2) (width 0.5) (layer "F.Cu") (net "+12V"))
 (segment (start 98.8 101) (end 94.4625 105.3375) (width 0.5) (layer "F.Cu") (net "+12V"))
 (segment (start 99.9 99.9) (end 98.8 101) (width 0.5) (layer "F.Cu") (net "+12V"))
 (segment (start 97.5 77.3) (end 82.3 77.3) (width 0.5) (layer "F.Cu") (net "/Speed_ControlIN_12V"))
 (segment (start 101.6 90.3) (end 100.7 89.4) (width 0.5) (layer "F.Cu") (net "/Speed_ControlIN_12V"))
 (segment (start 105 90.3) (end 101.6 90.3) (width 0.5) (layer "F.Cu") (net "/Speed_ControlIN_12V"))
 (segment (start 82.3 77.3) (end 81.2 78.4) (width 0.5) (layer "F.Cu") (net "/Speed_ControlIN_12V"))
 (segment (start 100.7 89.4) (end 100.7 80.5) (width 0.5) (layer "F.Cu") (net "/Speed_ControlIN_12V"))
 (segment (start 100.7 80.5) (end 97.5 77.3) (width 0.5) (layer "F.Cu") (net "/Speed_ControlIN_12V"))
 (segment (start 81.2 86.745) (end 74.445 93.5) (width 0.5) (layer "F.Cu") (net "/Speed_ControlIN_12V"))
 (segment (start 81.2 78.4) (end 81.2 86.745) (width 0.5) (layer "F.Cu") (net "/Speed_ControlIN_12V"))
 (segment (start 88.5 78.4) (end 84.1 78.4) (width 0.5) (layer "F.Cu") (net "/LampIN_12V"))
 (segment (start 89.75 79.65) (end 88.5 78.4) (width 0.5) (layer "F.Cu") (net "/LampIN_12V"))
 (segment (start 82.8 93.2) (end 80 96) (width 0.5) (layer "F.Cu") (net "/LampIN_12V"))
 (segment (start 89.925 81.125) (end 89.75 81.3) (width 0.5) (layer "F.Cu") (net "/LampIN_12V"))
 (segment (start 84.1 78.4) (end 82.8 79.7) (width 0.5) (layer "F.Cu") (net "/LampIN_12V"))
 (segment (start 82.8 79.7) (end 82.8 93.2) (width 0.5) (layer "F.Cu") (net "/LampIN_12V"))
 (segment (start 80 96) (end 74.445 96) (width 0.5) (layer "F.Cu") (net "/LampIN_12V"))
 (segment (start 94.0375 81.125) (end 89.925 81.125) (width 0.5) (layer "F.Cu") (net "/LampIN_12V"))
 (segment (start 89.75 81.3) (end 89.75 79.65) (width 0.5) (layer "F.Cu") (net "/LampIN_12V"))
 (segment (start 88.5 93.9) (end 84.5 93.9) (width 0.5) (layer "F.Cu") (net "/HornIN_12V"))
 (segment (start 84.5 93.9) (end 79.9 98.5) (width 0.5) (layer "F.Cu") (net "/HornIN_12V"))
 (segment (start 89.8 92.6) (end 88.5 93.9) (width 0.5) (layer "F.Cu") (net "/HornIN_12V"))
 (segment (start 94.0375 89.725) (end 89.825 89.725) (width 0.5) (layer "F.Cu") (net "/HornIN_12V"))
 (segment (start 79.9 98.5) (end 74.445 98.5) (width 0.5) (layer "F.Cu") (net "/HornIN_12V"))
 (segment (start 89.825 89.725) (end 89.8 89.7) (width 0.5) (layer "F.Cu") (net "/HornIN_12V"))
 (segment (start 89.8 89.7) (end 89.8 92.6) (width 0.5) (layer "F.Cu") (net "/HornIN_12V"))
 (segment (start 86.6 103.5125) (end 86.6 97.9) (width 0.5) (layer "F.Cu") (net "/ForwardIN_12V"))
 (segment (start 86.6 97.9) (end 86.7 97.8) (width 0.5) (layer "F.Cu") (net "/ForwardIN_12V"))
 (segment (start 83.9 103.5) (end 74.445 103.5) (width 0.5) (layer "F.Cu") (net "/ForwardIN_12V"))
 (segment (start 86.6 103.5125) (end 83.9125 103.5125) (width 0.5) (layer "F.Cu") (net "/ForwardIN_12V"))
 (segment (start 84.975 96.025) (end 88.3 96.025) (width 0.5) (layer "F.Cu") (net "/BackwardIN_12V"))
 (segment (start 83.7 97.3) (end 84.975 96.025) (width 0.5) (layer "F.Cu") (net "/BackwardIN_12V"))
 (segment (start 82.2 101) (end 83.7 99.5) (width 0.5) (layer "F.Cu") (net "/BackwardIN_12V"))
 (segment (start 89.3 97.9) (end 89.2 97.8) (width 0.5) (layer "F.Cu") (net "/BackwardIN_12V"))
 (segment (start 88.3 96.025) (end 89.2 96.925) (width 0.5) (layer "F.Cu") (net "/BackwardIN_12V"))
 (segment (start 89.3 103.5125) (end 89.3 97.9) (width 0.5) (layer "F.Cu") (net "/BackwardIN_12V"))
 (segment (start 89.2 96.925) (end 89.2 97.8) (width 0.5) (layer "F.Cu") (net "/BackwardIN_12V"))
 (segment (start 74.445 101) (end 82.2 101) (width 0.5) (layer "F.Cu") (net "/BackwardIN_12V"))
 (segment (start 83.7 99.5) (end 83.7 97.3) (width 0.5) (layer "F.Cu") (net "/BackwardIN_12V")))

